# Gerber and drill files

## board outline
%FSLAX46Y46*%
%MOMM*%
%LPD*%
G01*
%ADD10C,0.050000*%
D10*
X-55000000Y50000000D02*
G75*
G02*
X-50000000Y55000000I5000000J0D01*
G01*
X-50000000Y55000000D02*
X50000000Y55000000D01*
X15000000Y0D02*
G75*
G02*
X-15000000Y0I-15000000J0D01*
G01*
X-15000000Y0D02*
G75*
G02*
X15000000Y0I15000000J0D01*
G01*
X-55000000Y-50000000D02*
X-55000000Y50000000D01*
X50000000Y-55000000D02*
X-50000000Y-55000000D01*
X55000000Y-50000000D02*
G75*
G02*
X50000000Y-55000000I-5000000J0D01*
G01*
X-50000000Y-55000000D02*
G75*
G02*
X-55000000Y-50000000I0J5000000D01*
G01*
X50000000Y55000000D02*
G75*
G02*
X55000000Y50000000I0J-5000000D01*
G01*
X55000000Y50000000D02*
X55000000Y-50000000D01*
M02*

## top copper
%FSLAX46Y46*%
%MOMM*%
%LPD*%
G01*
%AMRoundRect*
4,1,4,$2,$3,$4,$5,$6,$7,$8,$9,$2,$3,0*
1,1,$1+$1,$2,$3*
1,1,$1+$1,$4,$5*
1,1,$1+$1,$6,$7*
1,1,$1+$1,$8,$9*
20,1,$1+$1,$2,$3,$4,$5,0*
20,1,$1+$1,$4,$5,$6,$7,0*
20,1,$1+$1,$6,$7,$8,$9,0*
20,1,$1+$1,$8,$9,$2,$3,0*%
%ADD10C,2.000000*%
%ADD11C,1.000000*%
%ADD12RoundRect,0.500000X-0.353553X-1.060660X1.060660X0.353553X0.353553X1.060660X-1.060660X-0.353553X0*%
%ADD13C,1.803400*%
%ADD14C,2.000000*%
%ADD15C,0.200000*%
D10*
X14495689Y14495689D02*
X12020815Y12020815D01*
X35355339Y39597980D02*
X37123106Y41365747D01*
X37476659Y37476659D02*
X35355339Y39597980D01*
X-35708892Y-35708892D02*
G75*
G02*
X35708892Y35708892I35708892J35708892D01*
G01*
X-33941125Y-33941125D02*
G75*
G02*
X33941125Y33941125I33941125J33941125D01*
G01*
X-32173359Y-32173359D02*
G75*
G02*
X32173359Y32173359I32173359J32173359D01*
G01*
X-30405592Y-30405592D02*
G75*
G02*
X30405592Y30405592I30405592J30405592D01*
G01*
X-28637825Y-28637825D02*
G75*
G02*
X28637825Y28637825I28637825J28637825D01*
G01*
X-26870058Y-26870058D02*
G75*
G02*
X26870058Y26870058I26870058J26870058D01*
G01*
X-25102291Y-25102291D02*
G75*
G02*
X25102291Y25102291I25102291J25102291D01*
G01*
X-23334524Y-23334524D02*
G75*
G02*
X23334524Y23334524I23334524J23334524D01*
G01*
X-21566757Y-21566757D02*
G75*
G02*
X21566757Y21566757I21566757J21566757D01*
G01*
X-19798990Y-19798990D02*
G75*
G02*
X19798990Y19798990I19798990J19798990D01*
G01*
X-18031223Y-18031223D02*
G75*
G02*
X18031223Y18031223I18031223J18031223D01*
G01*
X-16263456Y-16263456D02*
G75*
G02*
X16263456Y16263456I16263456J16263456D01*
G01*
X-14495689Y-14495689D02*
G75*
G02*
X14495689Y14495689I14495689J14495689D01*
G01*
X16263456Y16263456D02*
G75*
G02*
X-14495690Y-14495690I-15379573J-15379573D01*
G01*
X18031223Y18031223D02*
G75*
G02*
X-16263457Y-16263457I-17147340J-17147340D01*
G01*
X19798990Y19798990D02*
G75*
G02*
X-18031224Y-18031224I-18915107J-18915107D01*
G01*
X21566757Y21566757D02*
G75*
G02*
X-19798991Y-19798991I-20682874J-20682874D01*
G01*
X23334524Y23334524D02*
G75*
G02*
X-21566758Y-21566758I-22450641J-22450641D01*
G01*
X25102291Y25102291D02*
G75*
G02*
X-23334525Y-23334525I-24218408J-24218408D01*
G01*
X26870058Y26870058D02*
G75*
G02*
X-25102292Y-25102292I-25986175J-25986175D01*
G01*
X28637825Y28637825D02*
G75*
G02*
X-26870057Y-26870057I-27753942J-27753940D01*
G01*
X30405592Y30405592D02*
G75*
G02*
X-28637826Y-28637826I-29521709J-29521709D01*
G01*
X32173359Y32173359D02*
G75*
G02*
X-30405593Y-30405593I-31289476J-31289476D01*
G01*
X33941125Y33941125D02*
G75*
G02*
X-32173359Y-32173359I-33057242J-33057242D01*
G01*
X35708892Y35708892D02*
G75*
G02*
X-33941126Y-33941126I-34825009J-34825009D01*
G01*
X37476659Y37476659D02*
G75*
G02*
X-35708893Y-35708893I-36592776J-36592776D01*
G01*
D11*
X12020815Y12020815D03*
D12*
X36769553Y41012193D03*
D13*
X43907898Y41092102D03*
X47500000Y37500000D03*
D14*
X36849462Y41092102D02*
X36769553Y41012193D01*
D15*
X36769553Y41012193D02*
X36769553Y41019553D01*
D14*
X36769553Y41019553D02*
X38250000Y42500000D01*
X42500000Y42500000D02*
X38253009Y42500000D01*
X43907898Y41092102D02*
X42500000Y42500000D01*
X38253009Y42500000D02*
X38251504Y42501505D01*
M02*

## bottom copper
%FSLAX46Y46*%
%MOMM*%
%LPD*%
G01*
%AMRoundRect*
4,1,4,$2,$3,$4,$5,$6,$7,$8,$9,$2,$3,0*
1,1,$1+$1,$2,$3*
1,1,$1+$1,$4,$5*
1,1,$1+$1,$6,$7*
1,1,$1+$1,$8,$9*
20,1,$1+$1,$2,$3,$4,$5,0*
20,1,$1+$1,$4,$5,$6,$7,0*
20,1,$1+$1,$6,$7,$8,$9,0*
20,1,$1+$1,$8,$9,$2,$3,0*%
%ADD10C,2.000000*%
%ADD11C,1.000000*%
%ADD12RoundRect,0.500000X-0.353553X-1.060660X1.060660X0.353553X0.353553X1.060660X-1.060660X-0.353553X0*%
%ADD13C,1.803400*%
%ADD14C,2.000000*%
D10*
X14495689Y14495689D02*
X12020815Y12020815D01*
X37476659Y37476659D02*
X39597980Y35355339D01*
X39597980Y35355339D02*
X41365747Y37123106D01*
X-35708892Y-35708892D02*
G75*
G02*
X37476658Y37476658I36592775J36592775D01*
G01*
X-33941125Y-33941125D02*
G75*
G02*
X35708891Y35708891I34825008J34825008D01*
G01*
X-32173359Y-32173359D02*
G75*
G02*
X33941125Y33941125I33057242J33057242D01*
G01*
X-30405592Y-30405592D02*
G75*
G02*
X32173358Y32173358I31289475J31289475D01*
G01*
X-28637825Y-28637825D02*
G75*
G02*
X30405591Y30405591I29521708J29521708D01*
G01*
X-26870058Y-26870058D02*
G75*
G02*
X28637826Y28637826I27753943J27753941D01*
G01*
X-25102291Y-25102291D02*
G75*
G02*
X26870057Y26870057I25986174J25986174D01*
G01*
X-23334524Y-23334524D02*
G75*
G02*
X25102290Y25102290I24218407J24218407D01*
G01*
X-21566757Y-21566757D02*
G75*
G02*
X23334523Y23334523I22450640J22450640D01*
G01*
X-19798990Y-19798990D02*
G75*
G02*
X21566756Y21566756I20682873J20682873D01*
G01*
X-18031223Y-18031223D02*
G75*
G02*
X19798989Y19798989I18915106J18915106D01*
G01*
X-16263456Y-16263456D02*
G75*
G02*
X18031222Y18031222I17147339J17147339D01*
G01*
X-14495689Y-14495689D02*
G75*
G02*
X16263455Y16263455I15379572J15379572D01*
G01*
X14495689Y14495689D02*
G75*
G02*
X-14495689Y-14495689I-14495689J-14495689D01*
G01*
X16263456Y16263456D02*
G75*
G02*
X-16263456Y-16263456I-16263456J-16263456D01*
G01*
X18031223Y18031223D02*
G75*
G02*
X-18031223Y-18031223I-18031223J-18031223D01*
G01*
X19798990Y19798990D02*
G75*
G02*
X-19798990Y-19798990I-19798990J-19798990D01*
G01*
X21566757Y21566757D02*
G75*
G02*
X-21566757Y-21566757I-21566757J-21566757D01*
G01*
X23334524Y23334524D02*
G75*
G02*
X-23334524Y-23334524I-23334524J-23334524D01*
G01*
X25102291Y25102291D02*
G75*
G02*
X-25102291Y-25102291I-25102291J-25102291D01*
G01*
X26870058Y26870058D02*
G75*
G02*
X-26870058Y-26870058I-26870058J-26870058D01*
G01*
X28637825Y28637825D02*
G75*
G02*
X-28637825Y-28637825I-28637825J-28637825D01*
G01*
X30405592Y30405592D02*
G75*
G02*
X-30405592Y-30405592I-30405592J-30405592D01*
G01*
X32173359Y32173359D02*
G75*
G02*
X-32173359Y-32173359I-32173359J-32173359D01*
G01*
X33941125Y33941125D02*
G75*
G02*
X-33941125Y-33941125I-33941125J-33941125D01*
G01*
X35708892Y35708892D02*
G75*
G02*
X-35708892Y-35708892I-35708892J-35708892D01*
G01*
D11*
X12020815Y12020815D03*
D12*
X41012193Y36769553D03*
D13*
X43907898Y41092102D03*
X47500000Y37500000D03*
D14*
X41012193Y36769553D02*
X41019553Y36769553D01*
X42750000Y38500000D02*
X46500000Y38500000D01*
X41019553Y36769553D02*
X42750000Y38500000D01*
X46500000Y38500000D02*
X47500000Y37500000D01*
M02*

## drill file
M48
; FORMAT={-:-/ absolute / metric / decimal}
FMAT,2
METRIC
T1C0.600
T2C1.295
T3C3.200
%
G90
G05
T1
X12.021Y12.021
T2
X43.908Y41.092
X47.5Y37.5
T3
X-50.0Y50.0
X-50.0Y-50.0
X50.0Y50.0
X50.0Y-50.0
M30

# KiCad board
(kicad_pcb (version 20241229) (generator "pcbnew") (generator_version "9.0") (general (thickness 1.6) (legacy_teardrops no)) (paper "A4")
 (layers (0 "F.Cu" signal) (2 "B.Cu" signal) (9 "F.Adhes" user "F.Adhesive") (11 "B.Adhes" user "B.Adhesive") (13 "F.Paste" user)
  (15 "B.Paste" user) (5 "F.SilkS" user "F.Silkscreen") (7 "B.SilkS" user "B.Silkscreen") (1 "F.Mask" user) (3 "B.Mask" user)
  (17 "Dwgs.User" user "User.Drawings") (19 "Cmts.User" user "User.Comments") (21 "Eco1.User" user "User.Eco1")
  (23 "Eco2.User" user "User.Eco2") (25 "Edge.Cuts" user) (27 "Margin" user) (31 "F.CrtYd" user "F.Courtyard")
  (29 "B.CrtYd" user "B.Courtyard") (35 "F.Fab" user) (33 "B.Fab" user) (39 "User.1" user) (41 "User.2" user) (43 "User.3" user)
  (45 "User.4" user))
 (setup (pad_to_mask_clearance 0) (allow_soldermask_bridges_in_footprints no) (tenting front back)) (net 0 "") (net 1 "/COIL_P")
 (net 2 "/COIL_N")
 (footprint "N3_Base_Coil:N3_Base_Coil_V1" (layer "F.Cu") (at 0 0 45)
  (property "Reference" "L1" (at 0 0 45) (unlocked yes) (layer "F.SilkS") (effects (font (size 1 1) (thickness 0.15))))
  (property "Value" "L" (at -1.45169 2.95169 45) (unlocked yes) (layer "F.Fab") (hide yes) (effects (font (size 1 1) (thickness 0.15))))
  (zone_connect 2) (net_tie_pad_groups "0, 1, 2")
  (fp_line (start 20.5 0) (end 17 0) (stroke (width 2) (type default)) (layer "F.Cu"))
  (fp_line (start 53 -3) (end 55.5 -3) (stroke (width 2) (type default)) (layer "F.Cu"))
  (fp_line (start 52.999999 0) (end 53 -3) (stroke (width 2) (type default)) (layer "F.Cu"))
  (fp_arc (start -50.499999 0) (mid 0 -50.499999) (end 50.499999 0) (stroke (width 2) (type default)) (layer "F.Cu"))
  (fp_arc (start -47.999999 0) (mid 0 -47.999999) (end 47.999999 0) (stroke (width 2) (type default)) (layer "F.Cu"))
  (fp_arc (start -45.500001 0) (mid 0 -45.500001) (end 45.500001 0) (stroke (width 2) (type default)) (layer "F.Cu"))
  (fp_arc (start -43.000001 0) (mid 0 -43.000001) (end 43.000001 0) (stroke (width 2) (type default)) (layer "F.Cu"))
  (fp_arc (start -40.500001 0) (mid 0 -40.500001) (end 40.500001 0) (stroke (width 2) (type default)) (layer "F.Cu"))
  (fp_arc (start -38 0) (mid 0 -38) (end 38 0) (stroke (width 2) (type default)) (layer "F.Cu"))
  (fp_arc (start -35.5 0) (mid 0 -35.5) (end 35.5 0) (stroke (width 2) (type default)) (layer "F.Cu"))
  (fp_arc (start -33 0) (mid 0 -33) (end 33 0) (stroke (width 2) (type default)) (layer "F.Cu"))
  (fp_arc (start -30.5 0) (mid 0 -30.5) (end 30.5 0) (stroke (width 2) (type default)) (layer "F.Cu"))
  (fp_arc (start -28 0) (mid 0 -28) (end 28 0) (stroke (width 2) (type default)) (layer "F.Cu"))
  (fp_arc (start -25.5 0) (mid 0 -25.5) (end 25.5 0) (stroke (width 2) (type default)) (layer "F.Cu"))
  (fp_arc (start -23 0) (mid 0 -23) (end 23 0) (stroke (width 2) (type default)) (layer "F.Cu"))
  (fp_arc (start -20.5 0) (mid 0 -20.5) (end 20.5 0) (stroke (width 2) (type default)) (layer "F.Cu"))
  (fp_arc (start 23 0) (mid 1.25 21.75) (end -20.5 0) (stroke (width 2) (type default)) (layer "F.Cu"))
  (fp_arc (start 25.5 0) (mid 1.25 24.25) (end -23 0) (stroke (width 2) (type default)) (layer "F.Cu"))
  (fp_arc (start 28 0) (mid 1.25 26.75) (end -25.5 0) (stroke (width 2) (type default)) (layer "F.Cu"))
  (fp_arc (start 30.5 0) (mid 1.25 29.25) (end -28 0) (stroke (width 2) (type default)) (layer "F.Cu"))
  (fp_arc (start 33 0) (mid 1.25 31.75) (end -30.5 0) (stroke (width 2) (type default)) (layer "F.Cu"))
  (fp_arc (start 35.5 0) (mid 1.25 34.25) (end -33 0) (stroke (width 2) (type default)) (layer "F.Cu"))
  (fp_arc (start 38 0) (mid 1.25 36.75) (end -35.5 0) (stroke (width 2) (type default)) (layer "F.Cu"))
  (fp_arc (start 40.500001 0) (mid 1.25 39.25) (end -38 0) (stroke (width 2) (type default)) (layer "F.Cu"))
  (fp_arc (start 43.000001 0) (mid 1.25 41.750001) (end -40.500001 0) (stroke (width 2) (type default)) (layer "F.Cu"))
  (fp_arc (start 45.500001 0) (mid 1.25 44.250001) (end -43.000001 0) (stroke (width 2) (type default)) (layer "F.Cu"))
  (fp_arc (start 47.999999 0) (mid 1.249999 46.75) (end -45.500001 0) (stroke (width 2) (type default)) (layer "F.Cu"))
  (fp_arc (start 50.499999 0) (mid 1.25 49.249999) (end -47.999999 0) (stroke (width 2) (type default)) (layer "F.Cu"))
  (fp_arc (start 52.999999 0) (mid 1.25 51.749999) (end -50.499999 0) (stroke (width 2) (type default)) (layer "F.Cu"))
  (fp_line (start 20.5 0) (end 17 0) (stroke (width 2) (type default)) (layer "B.Cu"))
  (fp_line (start 52.999999 0) (end 53 3) (stroke (width 2) (type default)) (layer "B.Cu"))
  (fp_line (start 53 3) (end 55.5 3) (stroke (width 2) (type default)) (layer "B.Cu"))
  (fp_arc (start -50.499999 0) (mid 1.25 -51.749999) (end 52.999999 0) (stroke (width 2) (type default)) (layer "B.Cu"))
  (fp_arc (start -47.999999 0) (mid 1.25 -49.249999) (end 50.499999 0) (stroke (width 2) (type default)) (layer "B.Cu"))
  (fp_arc (start -45.500001 0) (mid 1.249999 -46.75) (end 47.999999 0) (stroke (width 2) (type default)) (layer "B.Cu"))
  (fp_arc (start -43.000001 0) (mid 1.25 -44.250001) (end 45.500001 0) (stroke (width 2) (type default)) (layer "B.Cu"))
  (fp_arc (start -40.500001 0) (mid 1.25 -41.750001) (end 43.000001 0) (stroke (width 2) (type default)) (layer "B.Cu"))
  (fp_arc (start -38 0) (mid 1.25 -39.25) (end 40.500001 0) (stroke (width 2) (type default)) (layer "B.Cu"))
  (fp_arc (start -35.5 0) (mid 1.25 -36.75) (end 38 0) (stroke (width 2) (type default)) (layer "B.Cu"))
  (fp_arc (start -33 0) (mid 1.25 -34.25) (end 35.5 0) (stroke (width 2) (type default)) (layer "B.Cu"))
  (fp_arc (start -30.5 0) (mid 1.25 -31.75) (end 33 0) (stroke (width 2) (type default)) (layer "B.Cu"))
  (fp_arc (start -28 0) (mid 1.25 -29.25) (end 30.5 0) (stroke (width 2) (type default)) (layer "B.Cu"))
  (fp_arc (start -25.5 0) (mid 1.25 -26.75) (end 28 0) (stroke (width 2) (type default)) (layer "B.Cu"))
  (fp_arc (start -23 0) (mid 1.25 -24.25) (end 25.5 0) (stroke (width 2) (type default)) (layer "B.Cu"))
  (fp_arc (start -20.5 0) (mid 1.25 -21.75) (end 23 0) (stroke (width 2) (type default)) (layer "B.Cu"))
  (fp_arc (start 20.5 0) (mid 0 20.5) (end -20.5 0) (stroke (width 2) (type default)) (layer "B.Cu"))
  (fp_arc (start 23 0) (mid 0 23) (end -23 0) (stroke (width 2) (type default)) (layer "B.Cu"))
  (fp_arc (start 25.5 0) (mid 0 25.5) (end -25.5 0) (stroke (width 2) (type default)) (layer "B.Cu"))
  (fp_arc (start 28 0) (mid 0 28) (end -28 0) (stroke (width 2) (type default)) (layer "B.Cu"))
  (fp_arc (start 30.5 0) (mid 0 30.5) (end -30.5 0) (stroke (width 2) (type default)) (layer "B.Cu"))
  (fp_arc (start 33 0) (mid 0 33) (end -33 0) (stroke (width 2) (type default)) (layer "B.Cu"))
  (fp_arc (start 35.5 0) (mid 0 35.5) (end -35.5 0) (stroke (width 2) (type default)) (layer "B.Cu"))
  (fp_arc (start 38 0) (mid 0 38) (end -38 0) (stroke (width 2) (type default)) (layer "B.Cu"))
  (fp_arc (start 40.500001 0) (mid 0 40.500001) (end -40.500001 0) (stroke (width 2) (type default)) (layer "B.Cu"))
  (fp_arc (start 43.000001 0) (mid 0 43.000001) (end -43.000001 0) (stroke (width 2) (type default)) (layer "B.Cu"))
  (fp_arc (start 45.500001 0) (mid 0 45.500001) (end -45.500001 0) (stroke (width 2) (type default)) (layer "B.Cu"))
  (fp_arc (start 47.999999 0) (mid 0 47.999999) (end -47.999999 0) (stroke (width 2) (type default)) (layer "B.Cu"))
  (fp_arc (start 50.499999 0) (mid 0 50.499999) (end -50.499999 0) (stroke (width 2) (type default)) (layer "B.Cu"))
  (pad "0" thru_hole circle (at 17 0 45) (size 1 1) (drill 0.6) (layers "*.Cu") (remove_unused_layers yes) (keep_end_layers yes)
   (zone_layer_connections))
  (pad "1" smd roundrect (at 55 -3 45) (size 3 2) (layers "F.Cu") (roundrect_rratio 0.25) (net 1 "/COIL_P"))
  (pad "2" smd roundrect (at 55 3 45) (size 3 2) (layers "B.Cu") (roundrect_rratio 0.25) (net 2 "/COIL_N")))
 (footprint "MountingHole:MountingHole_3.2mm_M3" (layer "F.Cu") (at 50 -50)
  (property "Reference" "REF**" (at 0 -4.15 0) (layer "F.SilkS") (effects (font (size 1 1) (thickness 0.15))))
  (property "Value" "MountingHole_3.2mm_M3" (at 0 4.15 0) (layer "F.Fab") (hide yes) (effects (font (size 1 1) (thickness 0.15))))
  (pad "" np_thru_hole circle (at 0 0) (size 3.2 3.2) (drill 3.2) (layers "*.Cu" "*.Mask")))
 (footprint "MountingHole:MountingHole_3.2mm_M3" (layer "F.Cu") (at -50 -50)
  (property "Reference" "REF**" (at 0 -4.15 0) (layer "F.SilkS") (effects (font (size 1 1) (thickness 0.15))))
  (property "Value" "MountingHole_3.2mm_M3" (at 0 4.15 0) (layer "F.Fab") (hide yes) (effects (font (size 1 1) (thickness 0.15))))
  (pad "" np_thru_hole circle (at 0 0) (size 3.2 3.2) (drill 3.2) (layers "*.Cu" "*.Mask")))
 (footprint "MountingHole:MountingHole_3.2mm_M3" (layer "F.Cu") (at 50 50)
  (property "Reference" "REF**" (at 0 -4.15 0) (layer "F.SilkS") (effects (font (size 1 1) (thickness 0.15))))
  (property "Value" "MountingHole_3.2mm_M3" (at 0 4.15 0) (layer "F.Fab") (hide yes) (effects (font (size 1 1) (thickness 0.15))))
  (pad "" np_thru_hole circle (at 0 0) (size 3.2 3.2) (drill 3.2) (layers "*.Cu" "*.Mask")))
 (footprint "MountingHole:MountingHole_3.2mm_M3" (layer "F.Cu") (at -50 50)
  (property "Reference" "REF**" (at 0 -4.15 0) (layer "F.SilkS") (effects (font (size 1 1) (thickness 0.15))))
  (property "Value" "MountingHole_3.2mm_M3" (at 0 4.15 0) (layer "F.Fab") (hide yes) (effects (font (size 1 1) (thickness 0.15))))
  (pad "" np_thru_hole circle (at 0 0) (size 3.2 3.2) (drill 3.2) (layers "*.Cu" "*.Mask")))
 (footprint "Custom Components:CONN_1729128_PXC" (layer "F.Cu") (at 43.907898 -41.092102 -45)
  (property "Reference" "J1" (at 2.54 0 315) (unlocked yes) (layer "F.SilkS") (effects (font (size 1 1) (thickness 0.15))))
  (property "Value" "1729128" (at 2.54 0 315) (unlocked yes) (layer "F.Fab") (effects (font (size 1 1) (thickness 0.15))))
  (pad "1" thru_hole circle (at 0 0 315) (size 1.8034 1.8034) (drill 1.2954) (layers "*.Cu" "*.Mask") (remove_unused_layers no)
   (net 1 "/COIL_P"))
  (pad "2" thru_hole circle (at 5.079999 0 315) (size 1.8034 1.8034) (drill 1.2954) (layers "*.Cu" "*.Mask") (remove_unused_layers no)
   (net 2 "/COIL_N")))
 (gr_arc (start -55 -50) (mid -53.535534 -53.535534) (end -50 -55) (stroke (width 0.05) (type default)) (locked yes) (layer "Edge.Cuts"))
 (gr_line (start -50 -55) (end 50 -55) (stroke (width 0.05) (type default)) (locked yes) (layer "Edge.Cuts"))
 (gr_circle (center 0 0) (end 15 0) (stroke (width 0.05) (type default)) (fill no) (locked yes) (layer "Edge.Cuts"))
 (gr_line (start -55 50) (end -55 -50) (stroke (width 0.05) (type default)) (locked yes) (layer "Edge.Cuts"))
 (gr_line (start 50 55) (end -50 55) (stroke (width 0.05) (type default)) (locked yes) (layer "Edge.Cuts"))
 (gr_arc (start 55 50) (mid 53.535534 53.535534) (end 50 55) (stroke (width 0.05) (type default)) (locked yes) (layer "Edge.Cuts"))
 (gr_arc (start -50 55) (mid -53.535534 53.535534) (end -55 50) (stroke (width 0.05) (type default)) (locked yes) (layer "Edge.Cuts"))
 (gr_arc (start 50 -55) (mid 53.535534 -53.535534) (end 55 -50) (stroke (width 0.05) (type default)) (locked yes) (layer "Edge.Cuts"))
 (gr_line (start 55 -50) (end 55 50) (stroke (width 0.05) (type default)) (locked yes) (layer "Edge.Cuts"))
 (segment (start 36.849462 -41.092102) (end 36.769553 -41.012193) (width 2) (layer "F.Cu") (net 1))
 (segment (start 36.769553 -41.012193) (end 36.769553 -41.019553) (width 0.2) (layer "F.Cu") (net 1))
 (segment (start 36.769553 -41.019553) (end 38.25 -42.5) (width 2) (layer "F.Cu") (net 1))
 (segment (start 42.5 -42.5) (end 38.253009 -42.5) (width 2) (layer "F.Cu") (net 1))
 (segment (start 43.907898 -41.092102) (end 42.5 -42.5) (width 2) (layer "F.Cu") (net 1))
 (segment (start 38.253009 -42.5) (end 38.251504 -42.501505) (width 2) (layer "F.Cu") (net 1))
 (segment (start 41.012193 -36.769553) (end 41.019553 -36.769553) (width 2) (layer "B.Cu") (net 2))
 (segment (start 42.75 -38.5) (end 46.5 -38.5) (width 2) (layer "B.Cu") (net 2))
 (segment (start 41.019553 -36.769553) (end 42.75 -38.5) (width 2) (layer "B.Cu") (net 2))
 (segment (start 46.5 -38.5) (end 47.5 -37.5) (width 2) (layer "B.Cu") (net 2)))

